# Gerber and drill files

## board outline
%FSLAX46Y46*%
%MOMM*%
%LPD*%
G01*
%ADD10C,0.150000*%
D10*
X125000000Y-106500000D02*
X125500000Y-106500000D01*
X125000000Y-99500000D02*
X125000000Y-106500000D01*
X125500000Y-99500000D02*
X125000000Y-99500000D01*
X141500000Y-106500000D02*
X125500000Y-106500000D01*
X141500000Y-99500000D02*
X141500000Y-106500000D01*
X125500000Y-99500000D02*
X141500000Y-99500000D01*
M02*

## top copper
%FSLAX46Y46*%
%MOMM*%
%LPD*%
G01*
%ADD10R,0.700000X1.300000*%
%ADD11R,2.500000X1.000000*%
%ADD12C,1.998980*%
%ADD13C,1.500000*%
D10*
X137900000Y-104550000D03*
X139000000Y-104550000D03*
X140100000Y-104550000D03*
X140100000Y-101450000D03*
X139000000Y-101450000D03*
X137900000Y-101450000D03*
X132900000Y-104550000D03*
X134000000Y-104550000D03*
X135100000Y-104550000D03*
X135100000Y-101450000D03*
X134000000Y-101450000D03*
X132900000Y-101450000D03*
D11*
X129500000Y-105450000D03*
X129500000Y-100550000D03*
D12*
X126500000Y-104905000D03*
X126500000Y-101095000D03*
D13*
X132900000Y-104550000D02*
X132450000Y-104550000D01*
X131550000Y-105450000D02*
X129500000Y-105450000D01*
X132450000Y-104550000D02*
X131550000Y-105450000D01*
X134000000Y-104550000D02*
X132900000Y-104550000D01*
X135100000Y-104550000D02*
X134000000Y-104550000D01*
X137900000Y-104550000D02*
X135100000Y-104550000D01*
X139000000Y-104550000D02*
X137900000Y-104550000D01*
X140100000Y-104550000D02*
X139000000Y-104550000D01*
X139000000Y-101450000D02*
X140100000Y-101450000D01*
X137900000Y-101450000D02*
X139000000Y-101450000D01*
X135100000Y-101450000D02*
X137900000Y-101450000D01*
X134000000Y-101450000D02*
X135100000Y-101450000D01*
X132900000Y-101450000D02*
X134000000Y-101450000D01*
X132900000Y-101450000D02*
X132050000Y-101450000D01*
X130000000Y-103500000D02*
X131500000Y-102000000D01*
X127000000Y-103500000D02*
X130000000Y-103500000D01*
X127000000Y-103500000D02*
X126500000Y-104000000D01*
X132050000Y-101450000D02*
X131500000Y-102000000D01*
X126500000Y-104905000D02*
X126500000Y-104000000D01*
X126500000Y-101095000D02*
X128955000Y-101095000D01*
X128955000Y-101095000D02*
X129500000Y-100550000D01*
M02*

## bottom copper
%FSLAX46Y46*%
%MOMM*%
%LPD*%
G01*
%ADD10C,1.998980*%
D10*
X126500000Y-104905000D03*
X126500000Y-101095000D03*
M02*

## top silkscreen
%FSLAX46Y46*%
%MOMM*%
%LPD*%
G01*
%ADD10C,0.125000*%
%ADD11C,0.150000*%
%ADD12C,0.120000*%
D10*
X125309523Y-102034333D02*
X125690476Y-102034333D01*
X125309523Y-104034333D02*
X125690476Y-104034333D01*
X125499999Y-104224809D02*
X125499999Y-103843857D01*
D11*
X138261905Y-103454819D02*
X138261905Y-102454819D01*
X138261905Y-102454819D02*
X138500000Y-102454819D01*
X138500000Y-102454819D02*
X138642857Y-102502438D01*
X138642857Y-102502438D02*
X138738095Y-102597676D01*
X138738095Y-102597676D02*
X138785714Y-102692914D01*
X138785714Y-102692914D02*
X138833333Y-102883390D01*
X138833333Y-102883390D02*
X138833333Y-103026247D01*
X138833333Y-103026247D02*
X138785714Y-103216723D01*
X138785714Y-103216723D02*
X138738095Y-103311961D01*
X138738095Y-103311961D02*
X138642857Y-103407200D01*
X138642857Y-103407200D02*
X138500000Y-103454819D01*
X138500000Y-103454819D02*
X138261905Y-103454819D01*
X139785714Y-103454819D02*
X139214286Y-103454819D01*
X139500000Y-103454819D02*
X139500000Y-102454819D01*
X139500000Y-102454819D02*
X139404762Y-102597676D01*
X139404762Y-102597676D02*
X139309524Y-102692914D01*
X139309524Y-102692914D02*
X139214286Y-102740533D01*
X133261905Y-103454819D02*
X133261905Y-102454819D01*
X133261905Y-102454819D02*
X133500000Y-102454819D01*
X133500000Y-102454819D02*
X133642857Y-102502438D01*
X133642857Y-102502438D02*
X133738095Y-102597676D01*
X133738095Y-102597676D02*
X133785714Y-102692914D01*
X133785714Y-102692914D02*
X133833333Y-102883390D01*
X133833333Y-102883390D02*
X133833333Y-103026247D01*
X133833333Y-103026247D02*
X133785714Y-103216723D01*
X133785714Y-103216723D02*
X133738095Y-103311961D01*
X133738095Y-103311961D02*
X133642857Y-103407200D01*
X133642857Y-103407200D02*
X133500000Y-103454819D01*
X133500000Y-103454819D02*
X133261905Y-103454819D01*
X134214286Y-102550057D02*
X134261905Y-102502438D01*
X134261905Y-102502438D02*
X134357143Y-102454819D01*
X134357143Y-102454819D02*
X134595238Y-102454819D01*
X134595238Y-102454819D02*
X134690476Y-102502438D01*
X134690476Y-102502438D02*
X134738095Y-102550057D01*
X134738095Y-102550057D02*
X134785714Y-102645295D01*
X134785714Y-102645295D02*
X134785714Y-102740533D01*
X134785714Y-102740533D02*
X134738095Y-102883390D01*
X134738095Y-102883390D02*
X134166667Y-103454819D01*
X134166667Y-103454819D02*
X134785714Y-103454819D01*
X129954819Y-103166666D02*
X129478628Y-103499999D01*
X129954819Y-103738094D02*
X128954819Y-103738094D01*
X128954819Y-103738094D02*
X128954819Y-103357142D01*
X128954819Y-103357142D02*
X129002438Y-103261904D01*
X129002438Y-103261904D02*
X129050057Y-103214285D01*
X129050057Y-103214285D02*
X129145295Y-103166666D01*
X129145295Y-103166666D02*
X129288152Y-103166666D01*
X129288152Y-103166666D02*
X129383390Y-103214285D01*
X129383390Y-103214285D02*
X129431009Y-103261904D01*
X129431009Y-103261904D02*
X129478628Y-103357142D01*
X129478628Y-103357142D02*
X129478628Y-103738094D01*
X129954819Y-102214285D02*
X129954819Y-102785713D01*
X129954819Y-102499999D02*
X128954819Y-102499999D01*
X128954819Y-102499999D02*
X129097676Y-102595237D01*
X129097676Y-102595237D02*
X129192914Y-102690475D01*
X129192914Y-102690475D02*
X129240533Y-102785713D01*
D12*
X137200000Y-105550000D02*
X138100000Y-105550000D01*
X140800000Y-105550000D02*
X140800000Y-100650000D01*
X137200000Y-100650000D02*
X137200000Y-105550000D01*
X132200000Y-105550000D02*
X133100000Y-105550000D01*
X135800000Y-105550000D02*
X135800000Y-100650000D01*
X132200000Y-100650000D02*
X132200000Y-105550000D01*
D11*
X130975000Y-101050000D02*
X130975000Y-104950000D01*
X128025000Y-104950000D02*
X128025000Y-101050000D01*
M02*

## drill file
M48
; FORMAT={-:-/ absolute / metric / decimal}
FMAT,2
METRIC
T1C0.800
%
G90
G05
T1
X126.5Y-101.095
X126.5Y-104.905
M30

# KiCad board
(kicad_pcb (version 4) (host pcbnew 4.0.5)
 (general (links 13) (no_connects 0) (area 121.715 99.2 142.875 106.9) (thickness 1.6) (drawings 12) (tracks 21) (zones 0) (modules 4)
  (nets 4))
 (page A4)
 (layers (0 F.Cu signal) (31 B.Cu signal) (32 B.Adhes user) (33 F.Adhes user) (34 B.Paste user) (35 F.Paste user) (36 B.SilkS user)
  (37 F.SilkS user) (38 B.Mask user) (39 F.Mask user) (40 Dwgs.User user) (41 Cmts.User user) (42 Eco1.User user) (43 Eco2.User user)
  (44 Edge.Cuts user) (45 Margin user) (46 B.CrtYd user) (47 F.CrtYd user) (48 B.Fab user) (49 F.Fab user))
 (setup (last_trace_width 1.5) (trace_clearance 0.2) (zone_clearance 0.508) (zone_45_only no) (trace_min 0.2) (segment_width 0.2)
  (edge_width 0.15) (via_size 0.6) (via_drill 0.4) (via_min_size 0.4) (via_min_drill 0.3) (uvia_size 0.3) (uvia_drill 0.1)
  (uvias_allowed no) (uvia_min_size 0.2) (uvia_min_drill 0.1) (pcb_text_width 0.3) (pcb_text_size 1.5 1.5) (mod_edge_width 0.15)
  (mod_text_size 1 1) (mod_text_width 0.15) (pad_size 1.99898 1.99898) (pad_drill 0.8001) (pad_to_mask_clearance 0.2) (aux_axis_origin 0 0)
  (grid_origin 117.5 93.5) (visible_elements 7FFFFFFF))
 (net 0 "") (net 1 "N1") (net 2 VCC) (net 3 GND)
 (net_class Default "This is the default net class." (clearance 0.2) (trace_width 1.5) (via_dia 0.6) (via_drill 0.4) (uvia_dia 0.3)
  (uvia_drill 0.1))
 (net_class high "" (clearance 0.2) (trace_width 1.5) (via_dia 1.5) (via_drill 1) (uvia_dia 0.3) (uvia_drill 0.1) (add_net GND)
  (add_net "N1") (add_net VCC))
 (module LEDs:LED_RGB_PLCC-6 (layer F.Cu) (at 139 103 90)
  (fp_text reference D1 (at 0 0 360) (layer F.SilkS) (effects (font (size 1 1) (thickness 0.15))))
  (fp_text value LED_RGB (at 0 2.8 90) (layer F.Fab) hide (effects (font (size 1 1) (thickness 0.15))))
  (fp_line (start -2.55 -1.8) (end -2.55 -0.9) (layer F.SilkS) (width 0.12))
  (fp_line (start -2.55 1.8) (end 2.35 1.8) (layer F.SilkS) (width 0.12))
  (fp_line (start 2.35 -1.8) (end -2.55 -1.8) (layer F.SilkS) (width 0.12))
  (pad 1 smd rect (at -1.55 -1.1 180) (size 0.7 1.3) (layers F.Cu F.Paste F.Mask) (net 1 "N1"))
  (pad 2 smd rect (at -1.55 0 180) (size 0.7 1.3) (layers F.Cu F.Paste F.Mask) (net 1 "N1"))
  (pad 3 smd rect (at -1.55 1.1 180) (size 0.7 1.3) (layers F.Cu F.Paste F.Mask) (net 1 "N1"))
  (pad 4 smd rect (at 1.55 1.1 180) (size 0.7 1.3) (layers F.Cu F.Paste F.Mask) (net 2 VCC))
  (pad 5 smd rect (at 1.55 0 180) (size 0.7 1.3) (layers F.Cu F.Paste F.Mask) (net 2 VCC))
  (pad 6 smd rect (at 1.55 -1.1 180) (size 0.7 1.3) (layers F.Cu F.Paste F.Mask) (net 2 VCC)))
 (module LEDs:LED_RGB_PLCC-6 (layer F.Cu) (at 134 103 90)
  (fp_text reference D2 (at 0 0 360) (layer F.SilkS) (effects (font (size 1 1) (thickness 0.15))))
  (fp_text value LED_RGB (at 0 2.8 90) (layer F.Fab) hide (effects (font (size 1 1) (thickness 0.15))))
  (fp_line (start -2.55 -1.8) (end -2.55 -0.9) (layer F.SilkS) (width 0.12))
  (fp_line (start -2.55 1.8) (end 2.35 1.8) (layer F.SilkS) (width 0.12))
  (fp_line (start 2.35 -1.8) (end -2.55 -1.8) (layer F.SilkS) (width 0.12))
  (pad 1 smd rect (at -1.55 -1.1 180) (size 0.7 1.3) (layers F.Cu F.Paste F.Mask) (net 1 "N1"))
  (pad 2 smd rect (at -1.55 0 180) (size 0.7 1.3) (layers F.Cu F.Paste F.Mask) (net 1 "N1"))
  (pad 3 smd rect (at -1.55 1.1 180) (size 0.7 1.3) (layers F.Cu F.Paste F.Mask) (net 1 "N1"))
  (pad 4 smd rect (at 1.55 1.1 180) (size 0.7 1.3) (layers F.Cu F.Paste F.Mask) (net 2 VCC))
  (pad 5 smd rect (at 1.55 0 180) (size 0.7 1.3) (layers F.Cu F.Paste F.Mask) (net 2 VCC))
  (pad 6 smd rect (at 1.55 -1.1 180) (size 0.7 1.3) (layers F.Cu F.Paste F.Mask) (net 2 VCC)))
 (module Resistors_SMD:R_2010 (layer F.Cu) (at 129.5 103 90)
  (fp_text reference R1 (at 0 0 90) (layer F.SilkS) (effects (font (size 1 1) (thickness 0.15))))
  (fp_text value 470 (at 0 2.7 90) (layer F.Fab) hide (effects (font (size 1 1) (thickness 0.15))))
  (fp_line (start 1.95 1.475) (end -1.95 1.475) (layer F.SilkS) (width 0.15))
  (fp_line (start -1.95 -1.475) (end 1.95 -1.475) (layer F.SilkS) (width 0.15))
  (pad 1 smd rect (at -2.45 0 90) (size 1 2.5) (layers F.Cu F.Paste F.Mask) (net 1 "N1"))
  (pad 2 smd rect (at 2.45 0 90) (size 1 2.5) (layers F.Cu F.Paste F.Mask) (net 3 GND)))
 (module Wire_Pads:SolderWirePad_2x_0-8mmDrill (layer F.Cu) (at 126.5 103 90)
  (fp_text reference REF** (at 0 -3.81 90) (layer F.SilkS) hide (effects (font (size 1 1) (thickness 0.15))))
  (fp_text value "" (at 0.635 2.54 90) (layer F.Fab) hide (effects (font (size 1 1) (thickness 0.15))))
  (pad 1 thru_hole circle (at -1.905 0 90) (size 1.99898 1.99898) (drill 0.8001) (layers *.Cu *.Mask) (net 2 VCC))
  (pad 2 thru_hole circle (at 1.905 0 90) (size 1.99898 1.99898) (drill 0.8001) (layers *.Cu *.Mask) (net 3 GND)))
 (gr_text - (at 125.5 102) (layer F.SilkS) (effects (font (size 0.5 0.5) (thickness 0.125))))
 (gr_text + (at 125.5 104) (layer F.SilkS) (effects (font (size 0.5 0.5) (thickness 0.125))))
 (gr_line (start 125 106.5) (end 125.5 106.5) (angle 90) (layer Edge.Cuts) (width 0.15))
 (gr_line (start 125 99.5) (end 125 106.5) (angle 90) (layer Edge.Cuts) (width 0.15))
 (gr_line (start 125.5 99.5) (end 125 99.5) (angle 90) (layer Edge.Cuts) (width 0.15))
 (gr_line (start 141.5 106.5) (end 125.5 106.5) (angle 90) (layer Edge.Cuts) (width 0.15))
 (gr_line (start 141.5 99.5) (end 141.5 106.5) (angle 90) (layer Edge.Cuts) (width 0.15))
 (gr_line (start 125.5 99.5) (end 141.5 99.5) (angle 90) (layer Edge.Cuts) (width 0.15))
 (segment (start 132.9 104.55) (end 132.45 104.55) (width 1.5) (layer F.Cu) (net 1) (status 400000))
 (segment (start 131.55 105.45) (end 129.5 105.45) (width 1.5) (layer F.Cu) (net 1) (status 800000))
 (segment (start 132.45 104.55) (end 131.55 105.45) (width 1.5) (layer F.Cu) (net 1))
 (segment (start 134 104.55) (end 132.9 104.55) (width 1.5) (layer F.Cu) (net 1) (status C00000))
 (segment (start 135.1 104.55) (end 134 104.55) (width 1.5) (layer F.Cu) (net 1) (status C00000))
 (segment (start 137.9 104.55) (end 135.1 104.55) (width 1.5) (layer F.Cu) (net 1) (status C00000))
 (segment (start 139 104.55) (end 137.9 104.55) (width 1.5) (layer F.Cu) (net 1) (status C00000))
 (segment (start 140.1 104.55) (end 139 104.55) (width 1.5) (layer F.Cu) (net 1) (status C00000))
 (segment (start 139 101.45) (end 140.1 101.45) (width 1.5) (layer F.Cu) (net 2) (status C00000))
 (segment (start 137.9 101.45) (end 139 101.45) (width 1.5) (layer F.Cu) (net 2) (status C00000))
 (segment (start 135.1 101.45) (end 137.9 101.45) (width 1.5) (layer F.Cu) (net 2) (status C00000))
 (segment (start 134 101.45) (end 135.1 101.45) (width 1.5) (layer F.Cu) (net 2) (status C00000))
 (segment (start 132.9 101.45) (end 134 101.45) (width 1.5) (layer F.Cu) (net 2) (status C00000))
 (segment (start 132.9 101.45) (end 132.05 101.45) (width 1.5) (layer F.Cu) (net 2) (status 400000))
 (segment (start 130 103.5) (end 131.5 102) (width 1.5) (layer F.Cu) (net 2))
 (segment (start 127 103.5) (end 130 103.5) (width 1.5) (layer F.Cu) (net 2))
 (segment (start 127 103.5) (end 126.5 104) (width 1.5) (layer F.Cu) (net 2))
 (segment (start 132.05 101.45) (end 131.5 102) (width 1.5) (layer F.Cu) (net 2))
 (segment (start 126.5 104.905) (end 126.5 104) (width 1.5) (layer F.Cu) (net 2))
 (segment (start 126.5 101.095) (end 128.955 101.095) (width 1.5) (layer F.Cu) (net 3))
 (segment (start 128.955 101.095) (end 129.5 100.55) (width 1.5) (layer F.Cu) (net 3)))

